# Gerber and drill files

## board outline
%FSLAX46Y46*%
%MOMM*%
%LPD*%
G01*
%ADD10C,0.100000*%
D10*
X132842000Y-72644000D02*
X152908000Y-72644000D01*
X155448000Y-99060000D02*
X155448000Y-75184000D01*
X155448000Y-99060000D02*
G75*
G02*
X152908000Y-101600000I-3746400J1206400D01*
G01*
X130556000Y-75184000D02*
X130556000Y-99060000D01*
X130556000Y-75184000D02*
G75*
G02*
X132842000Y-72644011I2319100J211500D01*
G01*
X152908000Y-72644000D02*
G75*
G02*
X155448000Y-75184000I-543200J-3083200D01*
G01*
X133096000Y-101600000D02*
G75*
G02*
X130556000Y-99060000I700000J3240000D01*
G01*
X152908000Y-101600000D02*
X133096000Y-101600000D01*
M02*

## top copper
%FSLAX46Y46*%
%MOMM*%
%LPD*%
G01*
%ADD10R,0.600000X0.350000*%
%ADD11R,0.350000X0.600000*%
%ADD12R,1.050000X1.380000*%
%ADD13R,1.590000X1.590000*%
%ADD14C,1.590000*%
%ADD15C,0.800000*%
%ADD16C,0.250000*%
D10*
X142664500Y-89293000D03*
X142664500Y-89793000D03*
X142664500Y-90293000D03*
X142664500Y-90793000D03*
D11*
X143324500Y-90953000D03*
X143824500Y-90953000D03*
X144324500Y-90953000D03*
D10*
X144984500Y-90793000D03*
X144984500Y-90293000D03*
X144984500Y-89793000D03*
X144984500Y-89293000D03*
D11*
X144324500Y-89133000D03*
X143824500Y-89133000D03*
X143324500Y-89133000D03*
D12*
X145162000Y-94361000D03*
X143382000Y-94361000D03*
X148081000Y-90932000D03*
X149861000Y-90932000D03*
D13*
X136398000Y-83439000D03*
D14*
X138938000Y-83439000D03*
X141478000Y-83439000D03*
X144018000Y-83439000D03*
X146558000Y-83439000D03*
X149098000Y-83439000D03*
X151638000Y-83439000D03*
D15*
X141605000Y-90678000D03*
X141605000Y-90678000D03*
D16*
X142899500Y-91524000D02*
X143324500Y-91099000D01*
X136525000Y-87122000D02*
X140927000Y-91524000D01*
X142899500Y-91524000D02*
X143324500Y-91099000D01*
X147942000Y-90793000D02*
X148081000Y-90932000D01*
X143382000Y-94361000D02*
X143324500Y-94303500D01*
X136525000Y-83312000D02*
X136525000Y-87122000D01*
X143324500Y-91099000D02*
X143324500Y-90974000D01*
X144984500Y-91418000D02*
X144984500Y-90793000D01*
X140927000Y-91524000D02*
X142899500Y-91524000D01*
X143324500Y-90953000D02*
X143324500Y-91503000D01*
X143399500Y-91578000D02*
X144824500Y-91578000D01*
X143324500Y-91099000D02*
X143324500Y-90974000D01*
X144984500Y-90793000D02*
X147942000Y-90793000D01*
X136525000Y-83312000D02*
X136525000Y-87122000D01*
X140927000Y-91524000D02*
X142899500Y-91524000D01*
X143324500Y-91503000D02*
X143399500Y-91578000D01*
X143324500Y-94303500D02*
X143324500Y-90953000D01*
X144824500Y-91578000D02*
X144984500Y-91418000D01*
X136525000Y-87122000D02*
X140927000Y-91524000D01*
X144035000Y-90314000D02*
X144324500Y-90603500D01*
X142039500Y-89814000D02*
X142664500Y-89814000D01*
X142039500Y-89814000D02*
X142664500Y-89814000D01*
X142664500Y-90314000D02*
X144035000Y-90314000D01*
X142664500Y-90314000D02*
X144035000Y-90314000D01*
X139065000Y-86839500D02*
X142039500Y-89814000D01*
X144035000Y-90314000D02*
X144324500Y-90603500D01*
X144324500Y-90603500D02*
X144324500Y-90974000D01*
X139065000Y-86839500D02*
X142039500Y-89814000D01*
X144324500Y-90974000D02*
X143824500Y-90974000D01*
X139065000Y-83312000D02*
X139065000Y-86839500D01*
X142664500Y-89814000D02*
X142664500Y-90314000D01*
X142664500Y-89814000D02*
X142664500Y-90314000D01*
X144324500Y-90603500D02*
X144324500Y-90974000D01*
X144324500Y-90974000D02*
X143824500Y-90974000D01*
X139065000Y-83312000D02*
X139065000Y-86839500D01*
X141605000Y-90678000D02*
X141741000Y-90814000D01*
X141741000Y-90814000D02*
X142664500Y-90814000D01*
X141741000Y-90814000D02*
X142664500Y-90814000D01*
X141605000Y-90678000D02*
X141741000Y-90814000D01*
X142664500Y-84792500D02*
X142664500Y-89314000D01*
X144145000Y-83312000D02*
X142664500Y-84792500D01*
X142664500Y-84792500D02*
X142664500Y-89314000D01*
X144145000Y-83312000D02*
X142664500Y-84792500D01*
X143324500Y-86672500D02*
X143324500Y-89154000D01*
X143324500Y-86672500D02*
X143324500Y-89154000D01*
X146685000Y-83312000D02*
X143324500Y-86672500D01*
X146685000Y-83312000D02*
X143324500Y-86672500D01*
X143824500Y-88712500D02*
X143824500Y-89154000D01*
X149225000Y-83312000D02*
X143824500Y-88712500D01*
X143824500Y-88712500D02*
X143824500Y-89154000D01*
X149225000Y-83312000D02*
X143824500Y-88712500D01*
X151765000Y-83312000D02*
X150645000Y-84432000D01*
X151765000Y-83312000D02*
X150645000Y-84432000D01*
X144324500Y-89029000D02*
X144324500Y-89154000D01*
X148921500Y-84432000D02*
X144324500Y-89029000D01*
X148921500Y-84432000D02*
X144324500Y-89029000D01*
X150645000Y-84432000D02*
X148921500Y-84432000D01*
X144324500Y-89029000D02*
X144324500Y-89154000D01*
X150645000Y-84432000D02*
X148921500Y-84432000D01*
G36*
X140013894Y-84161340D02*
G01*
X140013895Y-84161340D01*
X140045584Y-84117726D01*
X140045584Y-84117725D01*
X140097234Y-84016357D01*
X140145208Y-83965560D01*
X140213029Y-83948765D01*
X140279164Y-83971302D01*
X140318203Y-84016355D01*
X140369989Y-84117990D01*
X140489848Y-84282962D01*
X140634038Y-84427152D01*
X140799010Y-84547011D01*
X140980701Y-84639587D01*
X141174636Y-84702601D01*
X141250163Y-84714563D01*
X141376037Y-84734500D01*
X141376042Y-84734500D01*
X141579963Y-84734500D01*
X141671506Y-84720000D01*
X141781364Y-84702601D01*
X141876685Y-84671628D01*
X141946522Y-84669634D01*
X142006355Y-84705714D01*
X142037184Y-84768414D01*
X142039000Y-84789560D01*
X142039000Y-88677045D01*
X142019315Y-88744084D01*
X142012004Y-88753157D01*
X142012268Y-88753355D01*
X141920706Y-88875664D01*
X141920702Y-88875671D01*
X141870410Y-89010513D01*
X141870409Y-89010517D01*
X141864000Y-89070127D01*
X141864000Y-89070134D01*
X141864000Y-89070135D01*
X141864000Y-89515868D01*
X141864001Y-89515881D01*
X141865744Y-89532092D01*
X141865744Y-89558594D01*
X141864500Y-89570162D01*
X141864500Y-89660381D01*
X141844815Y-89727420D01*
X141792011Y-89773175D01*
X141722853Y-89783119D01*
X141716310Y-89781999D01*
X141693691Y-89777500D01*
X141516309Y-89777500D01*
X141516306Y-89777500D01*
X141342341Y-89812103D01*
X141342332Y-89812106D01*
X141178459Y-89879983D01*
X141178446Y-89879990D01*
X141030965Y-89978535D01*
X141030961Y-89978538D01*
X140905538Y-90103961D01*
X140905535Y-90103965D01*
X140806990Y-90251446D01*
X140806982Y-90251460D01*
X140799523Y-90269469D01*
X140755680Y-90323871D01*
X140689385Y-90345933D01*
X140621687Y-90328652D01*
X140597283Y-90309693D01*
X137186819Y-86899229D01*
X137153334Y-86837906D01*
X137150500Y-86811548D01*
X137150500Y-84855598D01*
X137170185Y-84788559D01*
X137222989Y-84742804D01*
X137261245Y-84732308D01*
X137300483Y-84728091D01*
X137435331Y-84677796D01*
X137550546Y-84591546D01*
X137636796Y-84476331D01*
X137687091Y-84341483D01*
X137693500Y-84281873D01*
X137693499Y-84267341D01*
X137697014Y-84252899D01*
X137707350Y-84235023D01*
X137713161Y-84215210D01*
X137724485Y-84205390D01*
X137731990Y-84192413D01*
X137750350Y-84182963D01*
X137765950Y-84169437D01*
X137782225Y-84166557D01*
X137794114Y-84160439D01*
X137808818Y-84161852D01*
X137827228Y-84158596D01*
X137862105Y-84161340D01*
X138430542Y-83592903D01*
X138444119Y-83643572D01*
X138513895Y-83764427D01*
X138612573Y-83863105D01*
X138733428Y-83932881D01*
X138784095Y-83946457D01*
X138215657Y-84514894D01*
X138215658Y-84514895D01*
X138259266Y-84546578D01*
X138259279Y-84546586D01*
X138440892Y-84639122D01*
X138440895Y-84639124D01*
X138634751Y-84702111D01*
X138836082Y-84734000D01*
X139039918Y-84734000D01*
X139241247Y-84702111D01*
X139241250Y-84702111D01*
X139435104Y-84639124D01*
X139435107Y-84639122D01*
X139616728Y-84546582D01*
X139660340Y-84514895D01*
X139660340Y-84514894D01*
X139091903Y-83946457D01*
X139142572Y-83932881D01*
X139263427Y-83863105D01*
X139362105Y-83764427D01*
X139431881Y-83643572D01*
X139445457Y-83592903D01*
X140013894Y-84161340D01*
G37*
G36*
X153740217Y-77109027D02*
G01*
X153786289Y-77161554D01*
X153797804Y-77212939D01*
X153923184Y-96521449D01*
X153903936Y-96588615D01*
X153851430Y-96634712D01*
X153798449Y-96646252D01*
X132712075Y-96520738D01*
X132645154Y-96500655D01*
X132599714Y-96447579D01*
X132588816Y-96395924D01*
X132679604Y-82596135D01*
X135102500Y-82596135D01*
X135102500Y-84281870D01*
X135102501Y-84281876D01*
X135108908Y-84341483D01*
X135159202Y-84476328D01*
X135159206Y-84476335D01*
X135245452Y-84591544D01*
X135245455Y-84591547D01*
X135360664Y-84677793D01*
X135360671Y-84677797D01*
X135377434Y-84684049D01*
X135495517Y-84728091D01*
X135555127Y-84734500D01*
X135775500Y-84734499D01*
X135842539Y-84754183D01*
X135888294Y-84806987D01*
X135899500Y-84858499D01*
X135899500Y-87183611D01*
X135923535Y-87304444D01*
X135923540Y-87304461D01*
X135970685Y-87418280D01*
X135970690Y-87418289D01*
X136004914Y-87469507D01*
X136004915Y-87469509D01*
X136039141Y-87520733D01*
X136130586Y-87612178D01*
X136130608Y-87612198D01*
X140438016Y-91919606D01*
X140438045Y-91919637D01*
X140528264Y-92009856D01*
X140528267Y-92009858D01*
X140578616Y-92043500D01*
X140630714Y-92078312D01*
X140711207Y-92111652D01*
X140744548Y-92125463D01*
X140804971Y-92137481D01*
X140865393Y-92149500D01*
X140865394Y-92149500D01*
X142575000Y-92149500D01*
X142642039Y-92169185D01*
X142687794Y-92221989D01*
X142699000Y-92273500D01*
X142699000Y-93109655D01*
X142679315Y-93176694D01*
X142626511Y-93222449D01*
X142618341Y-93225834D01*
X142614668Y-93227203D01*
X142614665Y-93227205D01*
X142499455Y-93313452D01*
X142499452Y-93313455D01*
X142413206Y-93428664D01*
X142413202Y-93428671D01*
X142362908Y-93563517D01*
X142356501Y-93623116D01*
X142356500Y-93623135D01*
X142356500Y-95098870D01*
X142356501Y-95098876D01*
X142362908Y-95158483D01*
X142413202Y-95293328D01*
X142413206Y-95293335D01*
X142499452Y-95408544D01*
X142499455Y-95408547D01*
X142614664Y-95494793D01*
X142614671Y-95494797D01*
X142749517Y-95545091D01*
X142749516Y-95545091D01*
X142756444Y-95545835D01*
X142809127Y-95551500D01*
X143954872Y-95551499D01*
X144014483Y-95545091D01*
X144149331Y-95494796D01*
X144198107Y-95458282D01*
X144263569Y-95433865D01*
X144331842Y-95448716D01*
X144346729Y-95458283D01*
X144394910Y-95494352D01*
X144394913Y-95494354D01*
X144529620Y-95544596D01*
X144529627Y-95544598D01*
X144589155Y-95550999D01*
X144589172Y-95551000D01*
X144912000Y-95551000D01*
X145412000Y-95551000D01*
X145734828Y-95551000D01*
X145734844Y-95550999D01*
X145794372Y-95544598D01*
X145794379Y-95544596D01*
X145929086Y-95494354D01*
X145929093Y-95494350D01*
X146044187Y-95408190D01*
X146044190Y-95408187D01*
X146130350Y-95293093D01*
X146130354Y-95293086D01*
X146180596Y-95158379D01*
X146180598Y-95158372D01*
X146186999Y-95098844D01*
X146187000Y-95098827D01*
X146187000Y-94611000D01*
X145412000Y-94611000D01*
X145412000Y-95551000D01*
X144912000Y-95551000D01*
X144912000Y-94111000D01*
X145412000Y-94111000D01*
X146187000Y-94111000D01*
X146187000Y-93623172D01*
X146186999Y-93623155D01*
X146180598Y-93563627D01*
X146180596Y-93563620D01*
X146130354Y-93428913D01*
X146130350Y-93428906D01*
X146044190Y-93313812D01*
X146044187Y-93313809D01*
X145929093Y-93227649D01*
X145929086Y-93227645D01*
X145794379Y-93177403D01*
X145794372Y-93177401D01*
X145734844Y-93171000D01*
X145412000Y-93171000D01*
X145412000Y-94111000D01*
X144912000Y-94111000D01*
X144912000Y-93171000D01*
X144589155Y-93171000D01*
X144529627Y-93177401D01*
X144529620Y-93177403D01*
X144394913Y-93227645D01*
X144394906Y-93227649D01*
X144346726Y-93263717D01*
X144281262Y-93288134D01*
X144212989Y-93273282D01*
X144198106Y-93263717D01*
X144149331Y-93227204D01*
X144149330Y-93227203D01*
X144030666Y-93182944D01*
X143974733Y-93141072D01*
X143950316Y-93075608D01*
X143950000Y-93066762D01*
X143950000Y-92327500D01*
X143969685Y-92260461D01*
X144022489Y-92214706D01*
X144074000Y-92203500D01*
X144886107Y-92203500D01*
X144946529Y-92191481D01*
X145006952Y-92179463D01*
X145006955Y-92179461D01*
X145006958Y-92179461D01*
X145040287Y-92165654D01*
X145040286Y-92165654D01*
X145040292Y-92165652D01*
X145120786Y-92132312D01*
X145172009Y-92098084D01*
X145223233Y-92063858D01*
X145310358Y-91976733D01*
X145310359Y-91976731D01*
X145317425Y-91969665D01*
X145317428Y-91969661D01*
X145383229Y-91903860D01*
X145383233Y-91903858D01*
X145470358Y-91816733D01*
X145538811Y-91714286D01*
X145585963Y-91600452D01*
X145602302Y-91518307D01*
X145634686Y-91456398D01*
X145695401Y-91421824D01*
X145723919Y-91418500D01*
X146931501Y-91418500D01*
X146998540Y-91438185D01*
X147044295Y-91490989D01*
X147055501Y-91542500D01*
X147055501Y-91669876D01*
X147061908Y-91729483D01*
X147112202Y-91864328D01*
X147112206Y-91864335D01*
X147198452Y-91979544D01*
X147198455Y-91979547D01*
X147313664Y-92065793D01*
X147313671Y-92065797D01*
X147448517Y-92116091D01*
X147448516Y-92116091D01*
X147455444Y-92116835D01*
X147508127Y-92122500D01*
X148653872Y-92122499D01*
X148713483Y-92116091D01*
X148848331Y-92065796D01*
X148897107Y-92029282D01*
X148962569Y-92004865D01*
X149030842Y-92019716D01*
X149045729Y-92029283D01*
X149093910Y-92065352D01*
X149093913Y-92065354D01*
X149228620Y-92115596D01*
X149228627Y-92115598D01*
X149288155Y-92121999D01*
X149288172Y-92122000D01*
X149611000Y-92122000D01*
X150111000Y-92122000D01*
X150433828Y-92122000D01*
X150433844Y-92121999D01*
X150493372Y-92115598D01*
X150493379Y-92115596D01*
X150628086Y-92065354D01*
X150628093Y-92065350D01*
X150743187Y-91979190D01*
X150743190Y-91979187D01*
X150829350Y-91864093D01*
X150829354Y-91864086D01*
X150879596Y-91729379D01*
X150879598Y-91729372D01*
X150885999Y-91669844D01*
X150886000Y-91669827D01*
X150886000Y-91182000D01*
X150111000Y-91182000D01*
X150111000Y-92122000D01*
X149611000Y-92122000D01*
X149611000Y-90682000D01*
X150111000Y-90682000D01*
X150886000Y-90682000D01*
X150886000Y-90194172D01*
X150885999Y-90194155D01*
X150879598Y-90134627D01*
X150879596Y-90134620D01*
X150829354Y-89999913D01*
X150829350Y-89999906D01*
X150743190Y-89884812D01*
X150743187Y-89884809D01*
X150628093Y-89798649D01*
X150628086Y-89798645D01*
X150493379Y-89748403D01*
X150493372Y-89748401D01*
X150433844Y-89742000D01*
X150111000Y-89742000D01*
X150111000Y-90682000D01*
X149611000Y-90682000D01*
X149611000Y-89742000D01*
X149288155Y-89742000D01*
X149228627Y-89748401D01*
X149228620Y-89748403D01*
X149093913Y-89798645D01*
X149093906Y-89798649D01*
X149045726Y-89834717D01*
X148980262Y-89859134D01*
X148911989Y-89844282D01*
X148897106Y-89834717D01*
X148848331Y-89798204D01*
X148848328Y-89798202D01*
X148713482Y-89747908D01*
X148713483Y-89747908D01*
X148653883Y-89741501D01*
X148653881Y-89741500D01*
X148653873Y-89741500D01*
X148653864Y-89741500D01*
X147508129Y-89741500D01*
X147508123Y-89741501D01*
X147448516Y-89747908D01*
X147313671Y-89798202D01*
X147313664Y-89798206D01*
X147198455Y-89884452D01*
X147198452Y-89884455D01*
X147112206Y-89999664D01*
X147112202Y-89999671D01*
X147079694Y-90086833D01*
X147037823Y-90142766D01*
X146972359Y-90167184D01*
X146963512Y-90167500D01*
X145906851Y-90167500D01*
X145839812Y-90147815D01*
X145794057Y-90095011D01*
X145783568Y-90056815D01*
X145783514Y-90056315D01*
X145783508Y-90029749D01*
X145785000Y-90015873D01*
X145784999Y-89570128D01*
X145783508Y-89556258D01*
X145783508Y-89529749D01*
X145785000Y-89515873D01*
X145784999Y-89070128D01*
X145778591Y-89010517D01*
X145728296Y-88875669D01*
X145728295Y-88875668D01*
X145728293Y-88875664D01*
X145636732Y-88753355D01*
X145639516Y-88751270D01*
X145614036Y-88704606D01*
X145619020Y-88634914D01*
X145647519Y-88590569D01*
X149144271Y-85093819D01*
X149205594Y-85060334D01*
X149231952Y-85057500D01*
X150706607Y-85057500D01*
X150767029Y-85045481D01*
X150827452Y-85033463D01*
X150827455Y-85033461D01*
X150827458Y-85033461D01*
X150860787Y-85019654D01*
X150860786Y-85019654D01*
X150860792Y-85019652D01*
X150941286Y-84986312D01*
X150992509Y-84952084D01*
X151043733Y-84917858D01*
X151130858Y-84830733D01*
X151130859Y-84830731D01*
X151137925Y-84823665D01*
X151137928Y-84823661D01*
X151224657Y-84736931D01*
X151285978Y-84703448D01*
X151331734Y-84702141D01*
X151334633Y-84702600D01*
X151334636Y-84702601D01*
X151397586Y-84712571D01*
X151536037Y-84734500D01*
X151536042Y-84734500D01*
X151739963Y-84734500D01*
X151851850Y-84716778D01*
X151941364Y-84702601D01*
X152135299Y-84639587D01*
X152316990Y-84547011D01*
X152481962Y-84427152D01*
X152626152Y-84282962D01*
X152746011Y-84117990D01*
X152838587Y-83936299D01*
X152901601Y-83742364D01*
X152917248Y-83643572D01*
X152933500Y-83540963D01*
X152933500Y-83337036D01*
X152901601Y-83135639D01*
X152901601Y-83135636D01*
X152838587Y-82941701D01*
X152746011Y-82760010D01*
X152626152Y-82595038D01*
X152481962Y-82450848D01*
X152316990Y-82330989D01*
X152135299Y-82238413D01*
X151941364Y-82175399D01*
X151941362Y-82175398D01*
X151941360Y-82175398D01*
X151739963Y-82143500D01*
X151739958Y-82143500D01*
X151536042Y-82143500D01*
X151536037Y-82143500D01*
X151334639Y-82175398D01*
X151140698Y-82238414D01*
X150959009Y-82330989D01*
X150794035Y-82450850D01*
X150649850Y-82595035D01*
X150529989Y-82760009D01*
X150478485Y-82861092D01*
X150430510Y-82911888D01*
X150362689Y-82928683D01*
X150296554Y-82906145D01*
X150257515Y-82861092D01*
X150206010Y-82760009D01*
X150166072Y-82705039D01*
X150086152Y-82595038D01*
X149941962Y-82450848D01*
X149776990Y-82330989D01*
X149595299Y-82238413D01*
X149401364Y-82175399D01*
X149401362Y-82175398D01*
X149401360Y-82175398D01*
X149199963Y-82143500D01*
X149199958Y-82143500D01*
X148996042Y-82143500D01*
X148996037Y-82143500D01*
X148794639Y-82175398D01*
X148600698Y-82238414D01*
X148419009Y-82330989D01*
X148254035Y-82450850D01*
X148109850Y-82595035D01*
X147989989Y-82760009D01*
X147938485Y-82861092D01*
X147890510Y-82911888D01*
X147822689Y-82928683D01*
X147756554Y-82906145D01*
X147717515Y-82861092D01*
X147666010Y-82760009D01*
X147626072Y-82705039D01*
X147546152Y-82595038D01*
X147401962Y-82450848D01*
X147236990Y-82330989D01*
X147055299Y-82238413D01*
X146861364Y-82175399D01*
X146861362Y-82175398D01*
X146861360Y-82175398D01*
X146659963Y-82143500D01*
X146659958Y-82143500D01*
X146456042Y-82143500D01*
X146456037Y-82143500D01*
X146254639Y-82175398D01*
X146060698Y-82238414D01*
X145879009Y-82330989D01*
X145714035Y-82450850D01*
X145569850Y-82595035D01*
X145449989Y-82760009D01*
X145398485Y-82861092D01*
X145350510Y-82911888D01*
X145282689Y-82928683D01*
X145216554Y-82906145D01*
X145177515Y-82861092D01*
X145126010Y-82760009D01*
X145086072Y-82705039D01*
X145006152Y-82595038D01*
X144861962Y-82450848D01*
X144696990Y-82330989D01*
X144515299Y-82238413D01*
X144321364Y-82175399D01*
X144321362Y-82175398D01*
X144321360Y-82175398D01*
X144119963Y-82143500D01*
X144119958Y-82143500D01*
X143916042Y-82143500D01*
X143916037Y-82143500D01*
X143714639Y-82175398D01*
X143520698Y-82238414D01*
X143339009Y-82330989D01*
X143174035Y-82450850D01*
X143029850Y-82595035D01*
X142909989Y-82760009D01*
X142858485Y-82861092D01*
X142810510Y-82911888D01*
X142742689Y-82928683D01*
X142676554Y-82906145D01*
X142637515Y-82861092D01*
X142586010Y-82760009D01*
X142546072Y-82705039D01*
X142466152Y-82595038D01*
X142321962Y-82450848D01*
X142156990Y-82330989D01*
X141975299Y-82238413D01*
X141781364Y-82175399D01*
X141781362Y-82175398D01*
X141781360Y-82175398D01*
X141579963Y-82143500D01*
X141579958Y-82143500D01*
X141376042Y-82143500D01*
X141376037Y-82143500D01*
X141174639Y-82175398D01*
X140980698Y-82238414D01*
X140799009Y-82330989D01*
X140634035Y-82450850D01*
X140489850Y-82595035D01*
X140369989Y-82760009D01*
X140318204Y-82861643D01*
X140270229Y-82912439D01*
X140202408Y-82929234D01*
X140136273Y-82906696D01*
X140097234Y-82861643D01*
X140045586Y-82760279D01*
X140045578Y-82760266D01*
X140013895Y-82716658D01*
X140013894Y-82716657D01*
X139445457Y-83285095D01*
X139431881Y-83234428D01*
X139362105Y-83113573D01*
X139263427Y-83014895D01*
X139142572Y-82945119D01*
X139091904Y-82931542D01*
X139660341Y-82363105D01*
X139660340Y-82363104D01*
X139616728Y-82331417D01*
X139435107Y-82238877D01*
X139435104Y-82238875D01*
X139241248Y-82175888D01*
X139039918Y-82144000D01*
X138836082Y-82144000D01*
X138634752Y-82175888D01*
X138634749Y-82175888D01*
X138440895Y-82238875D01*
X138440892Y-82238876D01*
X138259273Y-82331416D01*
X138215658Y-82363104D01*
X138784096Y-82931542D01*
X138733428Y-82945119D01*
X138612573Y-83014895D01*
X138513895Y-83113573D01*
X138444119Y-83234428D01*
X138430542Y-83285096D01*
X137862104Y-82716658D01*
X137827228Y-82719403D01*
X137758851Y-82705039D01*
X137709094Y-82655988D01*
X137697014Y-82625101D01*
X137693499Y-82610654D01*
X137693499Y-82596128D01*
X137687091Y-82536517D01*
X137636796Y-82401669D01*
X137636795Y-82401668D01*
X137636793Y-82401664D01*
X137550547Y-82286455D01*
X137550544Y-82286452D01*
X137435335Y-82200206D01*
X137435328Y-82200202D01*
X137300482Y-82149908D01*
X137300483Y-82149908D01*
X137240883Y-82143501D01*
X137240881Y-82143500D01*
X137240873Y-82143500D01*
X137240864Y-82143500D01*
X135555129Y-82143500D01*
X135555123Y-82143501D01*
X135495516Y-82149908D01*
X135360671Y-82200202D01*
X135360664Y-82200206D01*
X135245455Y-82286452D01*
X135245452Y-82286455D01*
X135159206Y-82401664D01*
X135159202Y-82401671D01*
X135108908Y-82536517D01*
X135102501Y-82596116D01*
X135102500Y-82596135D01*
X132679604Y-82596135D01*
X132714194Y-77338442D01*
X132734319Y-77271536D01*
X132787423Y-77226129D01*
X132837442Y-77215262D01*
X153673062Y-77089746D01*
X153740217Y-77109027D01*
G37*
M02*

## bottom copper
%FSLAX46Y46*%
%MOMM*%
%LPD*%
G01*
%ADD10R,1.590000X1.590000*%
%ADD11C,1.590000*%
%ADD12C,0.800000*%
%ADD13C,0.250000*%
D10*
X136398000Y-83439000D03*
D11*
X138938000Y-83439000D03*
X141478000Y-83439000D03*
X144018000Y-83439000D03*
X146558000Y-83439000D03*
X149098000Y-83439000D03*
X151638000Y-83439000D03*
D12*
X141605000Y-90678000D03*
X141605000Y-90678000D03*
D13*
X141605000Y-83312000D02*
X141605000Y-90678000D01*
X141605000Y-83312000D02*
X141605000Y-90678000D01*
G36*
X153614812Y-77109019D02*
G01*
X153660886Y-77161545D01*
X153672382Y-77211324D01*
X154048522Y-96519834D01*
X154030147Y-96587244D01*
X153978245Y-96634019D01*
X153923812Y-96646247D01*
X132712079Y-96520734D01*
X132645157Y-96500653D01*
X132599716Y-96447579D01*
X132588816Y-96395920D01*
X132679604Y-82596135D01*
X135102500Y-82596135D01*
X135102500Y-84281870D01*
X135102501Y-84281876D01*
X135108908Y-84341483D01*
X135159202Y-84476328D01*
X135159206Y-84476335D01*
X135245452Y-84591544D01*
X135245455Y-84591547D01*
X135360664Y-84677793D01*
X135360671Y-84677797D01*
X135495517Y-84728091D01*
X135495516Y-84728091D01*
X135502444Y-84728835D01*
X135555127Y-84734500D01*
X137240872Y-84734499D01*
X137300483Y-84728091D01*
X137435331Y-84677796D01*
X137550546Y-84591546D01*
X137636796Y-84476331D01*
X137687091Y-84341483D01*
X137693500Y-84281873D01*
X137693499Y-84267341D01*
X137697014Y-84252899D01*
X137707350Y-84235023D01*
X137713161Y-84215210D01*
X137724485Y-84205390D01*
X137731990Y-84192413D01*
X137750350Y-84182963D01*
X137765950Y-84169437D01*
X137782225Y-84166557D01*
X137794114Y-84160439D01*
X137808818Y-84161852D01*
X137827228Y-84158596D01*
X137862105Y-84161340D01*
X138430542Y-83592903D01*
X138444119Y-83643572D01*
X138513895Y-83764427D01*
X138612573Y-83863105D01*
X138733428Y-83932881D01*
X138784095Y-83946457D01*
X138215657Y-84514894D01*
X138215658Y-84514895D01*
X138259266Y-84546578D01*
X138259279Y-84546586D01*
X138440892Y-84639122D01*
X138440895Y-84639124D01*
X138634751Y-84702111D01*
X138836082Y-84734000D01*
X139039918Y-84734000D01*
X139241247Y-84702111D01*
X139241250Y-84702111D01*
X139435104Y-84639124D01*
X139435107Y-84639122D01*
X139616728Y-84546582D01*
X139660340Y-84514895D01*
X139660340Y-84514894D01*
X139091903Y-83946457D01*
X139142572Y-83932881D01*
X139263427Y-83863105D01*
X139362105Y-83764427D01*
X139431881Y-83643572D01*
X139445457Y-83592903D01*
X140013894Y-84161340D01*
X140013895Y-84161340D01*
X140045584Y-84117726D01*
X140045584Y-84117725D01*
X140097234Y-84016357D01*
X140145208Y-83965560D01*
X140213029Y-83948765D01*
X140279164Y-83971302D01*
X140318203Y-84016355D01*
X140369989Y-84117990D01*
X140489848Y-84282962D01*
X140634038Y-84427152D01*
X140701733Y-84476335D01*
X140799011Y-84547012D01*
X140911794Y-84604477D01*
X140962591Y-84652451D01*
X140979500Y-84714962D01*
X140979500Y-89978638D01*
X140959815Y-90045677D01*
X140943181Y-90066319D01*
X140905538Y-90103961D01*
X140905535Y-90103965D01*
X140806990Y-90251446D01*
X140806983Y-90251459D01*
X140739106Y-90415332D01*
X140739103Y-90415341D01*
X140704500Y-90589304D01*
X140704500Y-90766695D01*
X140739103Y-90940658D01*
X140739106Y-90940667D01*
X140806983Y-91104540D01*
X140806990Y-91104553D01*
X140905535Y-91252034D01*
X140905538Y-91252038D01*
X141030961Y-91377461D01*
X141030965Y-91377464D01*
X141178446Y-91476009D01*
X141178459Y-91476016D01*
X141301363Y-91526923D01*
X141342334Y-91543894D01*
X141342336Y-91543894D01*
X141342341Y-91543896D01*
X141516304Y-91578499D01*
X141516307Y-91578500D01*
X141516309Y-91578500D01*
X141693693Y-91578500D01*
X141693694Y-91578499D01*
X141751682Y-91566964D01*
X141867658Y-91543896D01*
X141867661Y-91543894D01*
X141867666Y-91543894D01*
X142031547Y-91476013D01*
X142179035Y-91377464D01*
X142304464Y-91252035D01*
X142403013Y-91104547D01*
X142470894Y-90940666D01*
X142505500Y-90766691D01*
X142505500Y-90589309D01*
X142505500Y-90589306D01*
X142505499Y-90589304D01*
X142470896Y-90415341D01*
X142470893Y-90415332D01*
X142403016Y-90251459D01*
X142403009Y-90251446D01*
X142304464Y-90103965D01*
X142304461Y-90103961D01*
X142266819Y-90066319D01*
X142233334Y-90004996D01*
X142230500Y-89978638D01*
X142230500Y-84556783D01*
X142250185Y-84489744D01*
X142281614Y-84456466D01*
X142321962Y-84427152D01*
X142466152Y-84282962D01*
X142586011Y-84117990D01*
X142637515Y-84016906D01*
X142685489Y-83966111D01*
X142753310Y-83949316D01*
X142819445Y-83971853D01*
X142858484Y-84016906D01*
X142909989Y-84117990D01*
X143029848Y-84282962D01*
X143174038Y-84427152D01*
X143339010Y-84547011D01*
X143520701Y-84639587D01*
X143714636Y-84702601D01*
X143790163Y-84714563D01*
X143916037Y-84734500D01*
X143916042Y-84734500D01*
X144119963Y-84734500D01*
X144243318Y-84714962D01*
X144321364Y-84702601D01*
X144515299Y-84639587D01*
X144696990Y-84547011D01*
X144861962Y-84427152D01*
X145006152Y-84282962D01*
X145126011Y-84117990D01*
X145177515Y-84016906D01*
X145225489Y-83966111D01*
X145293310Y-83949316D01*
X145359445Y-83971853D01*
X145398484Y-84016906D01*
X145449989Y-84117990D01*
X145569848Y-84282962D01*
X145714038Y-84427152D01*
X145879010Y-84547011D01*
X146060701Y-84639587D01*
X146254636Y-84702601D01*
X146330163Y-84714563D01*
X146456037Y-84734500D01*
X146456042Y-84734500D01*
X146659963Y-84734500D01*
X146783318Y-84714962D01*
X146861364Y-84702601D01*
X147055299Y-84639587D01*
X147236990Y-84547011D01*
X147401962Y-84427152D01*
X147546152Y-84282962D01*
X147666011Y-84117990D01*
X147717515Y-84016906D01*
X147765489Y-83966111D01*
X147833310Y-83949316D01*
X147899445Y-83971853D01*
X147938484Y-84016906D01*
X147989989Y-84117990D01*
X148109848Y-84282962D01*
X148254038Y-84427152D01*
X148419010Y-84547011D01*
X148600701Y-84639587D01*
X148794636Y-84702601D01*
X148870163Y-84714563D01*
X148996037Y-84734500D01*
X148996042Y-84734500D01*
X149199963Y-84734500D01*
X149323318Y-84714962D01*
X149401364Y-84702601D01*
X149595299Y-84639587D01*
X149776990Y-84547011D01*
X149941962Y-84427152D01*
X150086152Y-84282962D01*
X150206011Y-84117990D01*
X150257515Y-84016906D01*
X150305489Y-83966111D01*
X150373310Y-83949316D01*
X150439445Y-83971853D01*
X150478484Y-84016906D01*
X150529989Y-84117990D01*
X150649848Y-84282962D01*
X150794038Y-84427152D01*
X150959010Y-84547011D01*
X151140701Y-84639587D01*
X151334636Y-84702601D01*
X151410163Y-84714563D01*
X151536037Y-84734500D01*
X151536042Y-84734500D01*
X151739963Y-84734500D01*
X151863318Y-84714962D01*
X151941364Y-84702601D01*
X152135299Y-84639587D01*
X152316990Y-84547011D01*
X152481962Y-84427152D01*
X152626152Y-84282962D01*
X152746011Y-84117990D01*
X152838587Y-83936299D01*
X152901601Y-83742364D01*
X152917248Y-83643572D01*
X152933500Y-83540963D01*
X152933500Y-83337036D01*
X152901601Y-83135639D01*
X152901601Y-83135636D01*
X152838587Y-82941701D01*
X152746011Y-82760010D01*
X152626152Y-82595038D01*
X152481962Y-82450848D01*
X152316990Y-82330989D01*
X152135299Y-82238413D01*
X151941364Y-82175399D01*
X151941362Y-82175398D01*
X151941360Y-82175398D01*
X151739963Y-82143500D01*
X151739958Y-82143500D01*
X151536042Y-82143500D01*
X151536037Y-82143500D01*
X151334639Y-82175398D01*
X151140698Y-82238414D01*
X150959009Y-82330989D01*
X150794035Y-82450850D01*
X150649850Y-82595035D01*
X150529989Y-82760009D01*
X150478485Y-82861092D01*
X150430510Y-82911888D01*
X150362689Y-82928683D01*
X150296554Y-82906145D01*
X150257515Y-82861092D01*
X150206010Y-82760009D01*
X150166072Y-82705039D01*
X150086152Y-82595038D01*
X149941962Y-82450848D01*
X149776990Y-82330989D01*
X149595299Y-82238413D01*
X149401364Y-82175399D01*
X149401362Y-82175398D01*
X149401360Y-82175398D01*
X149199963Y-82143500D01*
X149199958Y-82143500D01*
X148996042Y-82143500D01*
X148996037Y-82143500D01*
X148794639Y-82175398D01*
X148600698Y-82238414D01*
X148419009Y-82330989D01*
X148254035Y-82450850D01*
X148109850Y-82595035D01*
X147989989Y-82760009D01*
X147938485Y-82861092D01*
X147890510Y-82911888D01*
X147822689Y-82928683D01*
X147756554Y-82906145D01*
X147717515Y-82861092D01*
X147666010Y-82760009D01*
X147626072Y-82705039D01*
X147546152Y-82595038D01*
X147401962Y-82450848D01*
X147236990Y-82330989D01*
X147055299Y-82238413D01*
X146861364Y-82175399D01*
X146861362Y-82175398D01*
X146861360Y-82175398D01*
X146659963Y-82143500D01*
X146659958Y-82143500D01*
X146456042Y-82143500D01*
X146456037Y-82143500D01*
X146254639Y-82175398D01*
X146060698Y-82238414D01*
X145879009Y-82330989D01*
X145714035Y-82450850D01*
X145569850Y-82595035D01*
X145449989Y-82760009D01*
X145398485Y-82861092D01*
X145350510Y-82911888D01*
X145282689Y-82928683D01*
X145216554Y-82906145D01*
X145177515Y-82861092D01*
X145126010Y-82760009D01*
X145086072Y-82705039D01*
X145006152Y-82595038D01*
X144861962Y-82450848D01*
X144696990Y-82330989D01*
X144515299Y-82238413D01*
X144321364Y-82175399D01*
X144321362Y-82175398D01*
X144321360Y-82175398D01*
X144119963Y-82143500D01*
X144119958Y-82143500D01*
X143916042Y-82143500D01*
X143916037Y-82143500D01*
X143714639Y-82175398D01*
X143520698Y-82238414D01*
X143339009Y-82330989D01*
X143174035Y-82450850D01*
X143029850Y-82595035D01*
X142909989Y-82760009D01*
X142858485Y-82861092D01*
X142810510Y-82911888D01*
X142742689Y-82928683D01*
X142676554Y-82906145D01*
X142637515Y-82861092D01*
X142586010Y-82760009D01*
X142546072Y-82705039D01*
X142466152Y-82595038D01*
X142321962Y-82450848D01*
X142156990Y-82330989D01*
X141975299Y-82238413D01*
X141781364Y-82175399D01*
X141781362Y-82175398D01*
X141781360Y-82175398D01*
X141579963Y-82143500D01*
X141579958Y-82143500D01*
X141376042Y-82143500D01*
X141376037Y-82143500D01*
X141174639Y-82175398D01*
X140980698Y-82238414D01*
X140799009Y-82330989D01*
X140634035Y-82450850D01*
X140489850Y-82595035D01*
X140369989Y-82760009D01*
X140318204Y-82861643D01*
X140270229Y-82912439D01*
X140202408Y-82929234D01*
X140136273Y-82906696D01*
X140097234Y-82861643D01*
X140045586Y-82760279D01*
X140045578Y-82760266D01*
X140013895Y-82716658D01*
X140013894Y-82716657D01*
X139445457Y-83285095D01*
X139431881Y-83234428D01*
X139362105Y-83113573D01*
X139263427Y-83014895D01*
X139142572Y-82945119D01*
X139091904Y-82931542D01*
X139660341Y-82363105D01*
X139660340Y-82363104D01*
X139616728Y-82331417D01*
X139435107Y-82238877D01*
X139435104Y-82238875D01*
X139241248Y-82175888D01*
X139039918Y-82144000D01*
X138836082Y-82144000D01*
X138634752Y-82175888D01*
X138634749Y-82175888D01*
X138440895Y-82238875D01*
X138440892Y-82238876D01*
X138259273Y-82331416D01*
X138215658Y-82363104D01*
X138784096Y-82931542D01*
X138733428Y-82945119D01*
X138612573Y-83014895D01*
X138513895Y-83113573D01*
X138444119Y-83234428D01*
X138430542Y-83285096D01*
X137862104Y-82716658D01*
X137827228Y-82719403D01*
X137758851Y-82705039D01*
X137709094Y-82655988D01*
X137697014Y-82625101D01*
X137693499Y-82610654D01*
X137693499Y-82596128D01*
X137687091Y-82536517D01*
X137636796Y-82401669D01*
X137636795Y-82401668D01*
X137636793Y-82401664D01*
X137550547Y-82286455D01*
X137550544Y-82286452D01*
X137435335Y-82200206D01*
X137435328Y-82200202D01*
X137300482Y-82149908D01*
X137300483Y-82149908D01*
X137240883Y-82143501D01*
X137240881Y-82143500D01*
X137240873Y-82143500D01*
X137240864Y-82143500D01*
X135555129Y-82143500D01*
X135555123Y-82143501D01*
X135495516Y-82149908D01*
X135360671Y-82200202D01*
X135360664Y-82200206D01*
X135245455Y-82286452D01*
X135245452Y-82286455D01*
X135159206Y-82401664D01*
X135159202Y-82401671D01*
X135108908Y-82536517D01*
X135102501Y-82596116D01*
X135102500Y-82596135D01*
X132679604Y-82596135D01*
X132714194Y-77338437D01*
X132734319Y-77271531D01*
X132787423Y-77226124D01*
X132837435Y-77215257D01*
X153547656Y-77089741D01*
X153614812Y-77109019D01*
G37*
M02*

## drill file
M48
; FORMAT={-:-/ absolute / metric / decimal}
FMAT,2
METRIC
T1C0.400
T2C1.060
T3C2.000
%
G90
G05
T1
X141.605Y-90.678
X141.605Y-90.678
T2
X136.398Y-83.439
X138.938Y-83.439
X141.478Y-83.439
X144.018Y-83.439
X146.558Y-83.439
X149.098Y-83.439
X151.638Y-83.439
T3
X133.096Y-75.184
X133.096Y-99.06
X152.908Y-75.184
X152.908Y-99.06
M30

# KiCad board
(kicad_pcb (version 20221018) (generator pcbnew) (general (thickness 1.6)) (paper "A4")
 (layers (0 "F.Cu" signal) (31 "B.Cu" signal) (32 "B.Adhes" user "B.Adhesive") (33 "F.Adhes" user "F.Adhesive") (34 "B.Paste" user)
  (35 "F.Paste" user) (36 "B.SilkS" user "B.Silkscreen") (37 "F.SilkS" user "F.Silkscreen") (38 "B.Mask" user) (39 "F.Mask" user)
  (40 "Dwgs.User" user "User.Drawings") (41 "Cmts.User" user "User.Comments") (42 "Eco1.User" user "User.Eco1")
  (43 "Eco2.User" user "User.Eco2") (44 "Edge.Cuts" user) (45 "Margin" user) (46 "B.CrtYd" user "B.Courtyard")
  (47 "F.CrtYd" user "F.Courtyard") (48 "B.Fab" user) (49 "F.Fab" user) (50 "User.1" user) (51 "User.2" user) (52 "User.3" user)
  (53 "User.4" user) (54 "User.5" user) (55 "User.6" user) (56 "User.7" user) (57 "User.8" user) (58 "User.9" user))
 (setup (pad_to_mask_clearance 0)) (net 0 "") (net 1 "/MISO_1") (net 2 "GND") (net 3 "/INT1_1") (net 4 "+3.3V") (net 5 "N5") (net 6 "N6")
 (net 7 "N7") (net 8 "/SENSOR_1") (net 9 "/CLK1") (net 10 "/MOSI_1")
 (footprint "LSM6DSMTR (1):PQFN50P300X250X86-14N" (layer "F.Cu") (at 143.8245 90.043)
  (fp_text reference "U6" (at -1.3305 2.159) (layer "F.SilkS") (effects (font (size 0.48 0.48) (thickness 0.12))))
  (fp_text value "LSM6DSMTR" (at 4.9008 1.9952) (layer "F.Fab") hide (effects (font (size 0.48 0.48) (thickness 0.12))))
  (pad "1" smd rect (at -1.16 -0.75) (size 0.6 0.35) (layers "F.Cu" "F.Paste" "F.Mask") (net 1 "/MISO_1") (solder_mask_margin 0.102))
  (pad "2" smd rect (at -1.16 -0.25) (size 0.6 0.35) (layers "F.Cu" "F.Paste" "F.Mask") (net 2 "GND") (solder_mask_margin 0.102))
  (pad "3" smd rect (at -1.16 0.25) (size 0.6 0.35) (layers "F.Cu" "F.Paste" "F.Mask") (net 2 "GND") (solder_mask_margin 0.102))
  (pad "4" smd rect (at -1.16 0.75) (size 0.6 0.35) (layers "F.Cu" "F.Paste" "F.Mask") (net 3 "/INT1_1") (solder_mask_margin 0.102))
  (pad "5" smd rect (at -0.5 0.91 90) (size 0.6 0.35) (layers "F.Cu" "F.Paste" "F.Mask") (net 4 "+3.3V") (solder_mask_margin 0.102))
  (pad "6" smd rect (at 0 0.91 90) (size 0.6 0.35) (layers "F.Cu" "F.Paste" "F.Mask") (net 2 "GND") (solder_mask_margin 0.102))
  (pad "7" smd rect (at 0.5 0.91 90) (size 0.6 0.35) (layers "F.Cu" "F.Paste" "F.Mask") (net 2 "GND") (solder_mask_margin 0.102))
  (pad "8" smd rect (at 1.16 0.75) (size 0.6 0.35) (layers "F.Cu" "F.Paste" "F.Mask") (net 4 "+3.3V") (solder_mask_margin 0.102))
  (pad "9" smd rect (at 1.16 0.25) (size 0.6 0.35) (layers "F.Cu" "F.Paste" "F.Mask") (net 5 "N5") (solder_mask_margin 0.102))
  (pad "10" smd rect (at 1.16 -0.25) (size 0.6 0.35) (layers "F.Cu" "F.Paste" "F.Mask") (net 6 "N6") (solder_mask_margin 0.102))
  (pad "11" smd rect (at 1.16 -0.75) (size 0.6 0.35) (layers "F.Cu" "F.Paste" "F.Mask") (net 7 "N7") (solder_mask_margin 0.102))
  (pad "12" smd rect (at 0.5 -0.91 90) (size 0.6 0.35) (layers "F.Cu" "F.Paste" "F.Mask") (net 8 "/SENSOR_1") (solder_mask_margin 0.102))
  (pad "13" smd rect (at 0 -0.91 90) (size 0.6 0.35) (layers "F.Cu" "F.Paste" "F.Mask") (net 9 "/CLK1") (solder_mask_margin 0.102))
  (pad "14" smd rect (at -0.5 -0.91 90) (size 0.6 0.35) (layers "F.Cu" "F.Paste" "F.Mask") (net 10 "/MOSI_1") (solder_mask_margin 0.102)))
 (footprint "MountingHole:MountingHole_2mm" (layer "F.Cu") (at 152.908 75.184)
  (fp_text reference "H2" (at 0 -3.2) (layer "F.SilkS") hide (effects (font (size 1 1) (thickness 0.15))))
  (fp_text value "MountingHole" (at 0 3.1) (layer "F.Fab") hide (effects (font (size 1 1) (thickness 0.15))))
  (pad "" np_thru_hole circle (at 0 0) (size 2 2) (drill 2) (layers "*.Cu" "*.Mask")))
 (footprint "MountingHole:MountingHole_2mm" (layer "F.Cu") (at 152.908 99.06)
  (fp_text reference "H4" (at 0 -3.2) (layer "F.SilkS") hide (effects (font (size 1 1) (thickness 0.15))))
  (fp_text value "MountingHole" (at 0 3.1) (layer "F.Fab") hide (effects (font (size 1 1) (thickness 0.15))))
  (pad "" np_thru_hole circle (at 0 0) (size 2 2) (drill 2) (layers "*.Cu" "*.Mask")))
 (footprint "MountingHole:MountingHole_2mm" (layer "F.Cu") (at 133.096 99.06)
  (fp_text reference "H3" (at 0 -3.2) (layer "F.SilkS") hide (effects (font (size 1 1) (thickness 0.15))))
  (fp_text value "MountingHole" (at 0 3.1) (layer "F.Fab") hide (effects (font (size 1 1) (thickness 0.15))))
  (pad "" np_thru_hole circle (at 0 0) (size 2 2) (drill 2) (layers "*.Cu" "*.Mask")))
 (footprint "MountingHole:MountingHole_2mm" (layer "F.Cu") (at 133.096 75.184)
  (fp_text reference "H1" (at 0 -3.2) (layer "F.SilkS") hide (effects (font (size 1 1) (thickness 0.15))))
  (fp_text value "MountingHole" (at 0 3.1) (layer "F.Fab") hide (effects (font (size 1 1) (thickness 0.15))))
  (pad "" np_thru_hole circle (at 0 0) (size 2 2) (drill 2) (layers "*.Cu" "*.Mask")))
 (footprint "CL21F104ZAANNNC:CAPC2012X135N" (layer "F.Cu") (at 144.272 94.361 180)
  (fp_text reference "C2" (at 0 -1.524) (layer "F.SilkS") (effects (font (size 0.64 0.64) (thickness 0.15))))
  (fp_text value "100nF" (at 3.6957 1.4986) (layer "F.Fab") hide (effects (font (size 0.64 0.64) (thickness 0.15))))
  (pad "1" smd rect (at -0.89 0 180) (size 1.05 1.38) (layers "F.Cu" "F.Paste" "F.Mask") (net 2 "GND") (solder_mask_margin 0.102))
  (pad "2" smd rect (at 0.89 0 180) (size 1.05 1.38) (layers "F.Cu" "F.Paste" "F.Mask") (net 4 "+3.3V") (solder_mask_margin 0.102)))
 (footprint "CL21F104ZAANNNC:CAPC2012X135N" (layer "F.Cu") (at 148.971 90.932)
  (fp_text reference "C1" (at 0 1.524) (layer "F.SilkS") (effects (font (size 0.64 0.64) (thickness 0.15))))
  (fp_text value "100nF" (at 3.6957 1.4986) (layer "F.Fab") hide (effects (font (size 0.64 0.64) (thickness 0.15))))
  (pad "1" smd rect (at -0.89 0) (size 1.05 1.38) (layers "F.Cu" "F.Paste" "F.Mask") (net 4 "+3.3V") (solder_mask_margin 0.102))
  (pad "2" smd rect (at 0.89 0) (size 1.05 1.38) (layers "F.Cu" "F.Paste" "F.Mask") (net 2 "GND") (solder_mask_margin 0.102)))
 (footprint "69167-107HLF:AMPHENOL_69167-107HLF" (layer "F.Cu") (at 144.018 83.439)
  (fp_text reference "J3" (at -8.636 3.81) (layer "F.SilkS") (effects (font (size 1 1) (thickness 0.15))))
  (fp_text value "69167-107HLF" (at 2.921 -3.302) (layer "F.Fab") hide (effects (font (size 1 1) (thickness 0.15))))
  (pad "01" thru_hole rect (at -7.62 0) (size 1.59 1.59) (drill 1.06) (layers "*.Cu" "*.Mask") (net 4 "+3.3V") (solder_mask_margin 0.102))
  (pad "02" thru_hole circle (at -5.08 0) (size 1.59 1.59) (drill 1.06) (layers "*.Cu" "*.Mask") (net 2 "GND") (solder_mask_margin 0.102))
  (pad "03" thru_hole circle (at -2.54 0) (size 1.59 1.59) (drill 1.06) (layers "*.Cu" "*.Mask") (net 3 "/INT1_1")
   (solder_mask_margin 0.102))
  (pad "04" thru_hole circle (at 0 0) (size 1.59 1.59) (drill 1.06) (layers "*.Cu" "*.Mask") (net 1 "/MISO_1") (solder_mask_margin 0.102))
  (pad "05" thru_hole circle (at 2.54 0) (size 1.59 1.59) (drill 1.06) (layers "*.Cu" "*.Mask") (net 10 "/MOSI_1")
   (solder_mask_margin 0.102))
  (pad "06" thru_hole circle (at 5.08 0) (size 1.59 1.59) (drill 1.06) (layers "*.Cu" "*.Mask") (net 9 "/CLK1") (solder_mask_margin 0.102))
  (pad "07" thru_hole circle (at 7.62 0) (size 1.59 1.59) (drill 1.06) (layers "*.Cu" "*.Mask") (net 8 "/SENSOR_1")
   (solder_mask_margin 0.102)))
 (gr_line (start 132.842 72.644) (end 152.908 72.644) (stroke (width 0.1) (type default)) (layer "Edge.Cuts"))
 (gr_line (start 155.448 99.06) (end 155.448 75.184) (stroke (width 0.1) (type default)) (layer "Edge.Cuts"))
 (gr_arc (start 155.448 99.06) (mid 154.484666 100.636666) (end 152.908 101.6) (stroke (width 0.1) (type default)) (layer "Edge.Cuts"))
 (gr_line (start 130.556 75.184) (end 130.556 99.06) (stroke (width 0.1) (type default)) (layer "Edge.Cuts"))
 (gr_arc (start 130.556 75.184) (mid 131.144178 73.41466) (end 132.842 72.644) (stroke (width 0.1) (type default)) (layer "Edge.Cuts"))
 (gr_arc (start 152.908 72.644) (mid 154.578529 73.513471) (end 155.448 75.184) (stroke (width 0.1) (type default)) (layer "Edge.Cuts"))
 (gr_arc (start 133.096 101.6) (mid 131.452114 100.703886) (end 130.556 99.06) (stroke (width 0.1) (type default)) (layer "Edge.Cuts"))
 (gr_line (start 152.908 101.6) (end 133.096 101.6) (stroke (width 0.1) (type default)) (layer "Edge.Cuts"))
 (segment (start 142.8995 91.524) (end 143.3245 91.099) (width 0.25) (layer "F.Cu") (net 4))
 (segment (start 136.525 87.122) (end 140.927 91.524) (width 0.25) (layer "F.Cu") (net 4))
 (segment (start 142.8995 91.524) (end 143.3245 91.099) (width 0.25) (layer "F.Cu") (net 4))
 (segment (start 147.942 90.793) (end 148.081 90.932) (width 0.25) (layer "F.Cu") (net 4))
 (segment (start 143.382 94.361) (end 143.3245 94.3035) (width 0.25) (layer "F.Cu") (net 4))
 (segment (start 136.525 83.312) (end 136.525 87.122) (width 0.25) (layer "F.Cu") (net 4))
 (segment (start 143.3245 91.099) (end 143.3245 90.974) (width 0.25) (layer "F.Cu") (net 4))
 (segment (start 144.9845 91.418) (end 144.9845 90.793) (width 0.25) (layer "F.Cu") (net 4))
 (segment (start 140.927 91.524) (end 142.8995 91.524) (width 0.25) (layer "F.Cu") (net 4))
 (segment (start 143.3245 90.953) (end 143.3245 91.503) (width 0.25) (layer "F.Cu") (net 4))
 (segment (start 143.3995 91.578) (end 144.8245 91.578) (width 0.25) (layer "F.Cu") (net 4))
 (segment (start 143.3245 91.099) (end 143.3245 90.974) (width 0.25) (layer "F.Cu") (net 4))
 (segment (start 144.9845 90.793) (end 147.942 90.793) (width 0.25) (layer "F.Cu") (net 4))
 (segment (start 136.525 83.312) (end 136.525 87.122) (width 0.25) (layer "F.Cu") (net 4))
 (segment (start 140.927 91.524) (end 142.8995 91.524) (width 0.25) (layer "F.Cu") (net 4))
 (segment (start 143.3245 91.503) (end 143.3995 91.578) (width 0.25) (layer "F.Cu") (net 4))
 (segment (start 143.3245 94.3035) (end 143.3245 90.953) (width 0.25) (layer "F.Cu") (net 4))
 (segment (start 144.8245 91.578) (end 144.9845 91.418) (width 0.25) (layer "F.Cu") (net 4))
 (segment (start 136.525 87.122) (end 140.927 91.524) (width 0.25) (layer "F.Cu") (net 4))
 (segment (start 144.035 90.314) (end 144.3245 90.6035) (width 0.25) (layer "F.Cu") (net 2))
 (segment (start 142.0395 89.814) (end 142.6645 89.814) (width 0.25) (layer "F.Cu") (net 2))
 (segment (start 142.0395 89.814) (end 142.6645 89.814) (width 0.25) (layer "F.Cu") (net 2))
 (segment (start 142.6645 90.314) (end 144.035 90.314) (width 0.25) (layer "F.Cu") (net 2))
 (segment (start 142.6645 90.314) (end 144.035 90.314) (width 0.25) (layer "F.Cu") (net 2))
 (segment (start 139.065 86.8395) (end 142.0395 89.814) (width 0.25) (layer "F.Cu") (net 2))
 (segment (start 144.035 90.314) (end 144.3245 90.6035) (width 0.25) (layer "F.Cu") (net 2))
 (segment (start 144.3245 90.6035) (end 144.3245 90.974) (width 0.25) (layer "F.Cu") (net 2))
 (segment (start 139.065 86.8395) (end 142.0395 89.814) (width 0.25) (layer "F.Cu") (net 2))
 (segment (start 144.3245 90.974) (end 143.8245 90.974) (width 0.25) (layer "F.Cu") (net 2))
 (segment (start 139.065 83.312) (end 139.065 86.8395) (width 0.25) (layer "F.Cu") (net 2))
 (segment (start 142.6645 89.814) (end 142.6645 90.314) (width 0.25) (layer "F.Cu") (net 2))
 (segment (start 142.6645 89.814) (end 142.6645 90.314) (width 0.25) (layer "F.Cu") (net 2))
 (segment (start 144.3245 90.6035) (end 144.3245 90.974) (width 0.25) (layer "F.Cu") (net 2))
 (segment (start 144.3245 90.974) (end 143.8245 90.974) (width 0.25) (layer "F.Cu") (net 2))
 (segment (start 139.065 83.312) (end 139.065 86.8395) (width 0.25) (layer "F.Cu") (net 2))
 (segment (start 141.605 90.678) (end 141.741 90.814) (width 0.25) (layer "F.Cu") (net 3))
 (segment (start 141.741 90.814) (end 142.6645 90.814) (width 0.25) (layer "F.Cu") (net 3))
 (segment (start 141.741 90.814) (end 142.6645 90.814) (width 0.25) (layer "F.Cu") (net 3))
 (segment (start 141.605 90.678) (end 141.741 90.814) (width 0.25) (layer "F.Cu") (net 3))
 (via (at 141.605 90.678) (size 0.8) (drill 0.4) (layers "F.Cu" "B.Cu") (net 3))
 (via (at 141.605 90.678) (size 0.8) (drill 0.4) (layers "F.Cu" "B.Cu") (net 3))
 (segment (start 141.605 83.312) (end 141.605 90.678) (width 0.25) (layer "B.Cu") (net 3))
 (segment (start 141.605 83.312) (end 141.605 90.678) (width 0.25) (layer "B.Cu") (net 3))
 (segment (start 142.6645 84.7925) (end 142.6645 89.314) (width 0.25) (layer "F.Cu") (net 1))
 (segment (start 144.145 83.312) (end 142.6645 84.7925) (width 0.25) (layer "F.Cu") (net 1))
 (segment (start 142.6645 84.7925) (end 142.6645 89.314) (width 0.25) (layer "F.Cu") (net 1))
 (segment (start 144.145 83.312) (end 142.6645 84.7925) (width 0.25) (layer "F.Cu") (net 1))
 (segment (start 143.3245 86.6725) (end 143.3245 89.154) (width 0.25) (layer "F.Cu") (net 10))
 (segment (start 143.3245 86.6725) (end 143.3245 89.154) (width 0.25) (layer "F.Cu") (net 10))
 (segment (start 146.685 83.312) (end 143.3245 86.6725) (width 0.25) (layer "F.Cu") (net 10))
 (segment (start 146.685 83.312) (end 143.3245 86.6725) (width 0.25) (layer "F.Cu") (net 10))
 (segment (start 143.8245 88.7125) (end 143.8245 89.154) (width 0.25) (layer "F.Cu") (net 9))
 (segment (start 149.225 83.312) (end 143.8245 88.7125) (width 0.25) (layer "F.Cu") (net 9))
 (segment (start 143.8245 88.7125) (end 143.8245 89.154) (width 0.25) (layer "F.Cu") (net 9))
 (segment (start 149.225 83.312) (end 143.8245 88.7125) (width 0.25) (layer "F.Cu") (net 9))
 (segment (start 151.765 83.312) (end 150.645 84.432) (width 0.25) (layer "F.Cu") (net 8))
 (segment (start 151.765 83.312) (end 150.645 84.432) (width 0.25) (layer "F.Cu") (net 8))
 (segment (start 144.3245 89.029) (end 144.3245 89.154) (width 0.25) (layer "F.Cu") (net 8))
 (segment (start 148.9215 84.432) (end 144.3245 89.029) (width 0.25) (layer "F.Cu") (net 8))
 (segment (start 148.9215 84.432) (end 144.3245 89.029) (width 0.25) (layer "F.Cu") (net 8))
 (segment (start 150.645 84.432) (end 148.9215 84.432) (width 0.25) (layer "F.Cu") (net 8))
 (segment (start 144.3245 89.029) (end 144.3245 89.154) (width 0.25) (layer "F.Cu") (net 8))
 (segment (start 150.645 84.432) (end 148.9215 84.432) (width 0.25) (layer "F.Cu") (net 8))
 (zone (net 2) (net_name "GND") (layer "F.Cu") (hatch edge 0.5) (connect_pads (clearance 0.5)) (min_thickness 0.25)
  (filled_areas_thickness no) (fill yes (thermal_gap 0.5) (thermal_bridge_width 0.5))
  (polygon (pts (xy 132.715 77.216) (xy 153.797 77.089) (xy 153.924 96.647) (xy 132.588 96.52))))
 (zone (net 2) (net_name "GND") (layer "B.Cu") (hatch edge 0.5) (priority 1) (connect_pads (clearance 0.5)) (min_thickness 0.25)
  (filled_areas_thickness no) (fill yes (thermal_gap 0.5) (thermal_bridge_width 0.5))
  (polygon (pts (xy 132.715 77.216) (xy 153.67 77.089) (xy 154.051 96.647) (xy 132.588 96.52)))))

